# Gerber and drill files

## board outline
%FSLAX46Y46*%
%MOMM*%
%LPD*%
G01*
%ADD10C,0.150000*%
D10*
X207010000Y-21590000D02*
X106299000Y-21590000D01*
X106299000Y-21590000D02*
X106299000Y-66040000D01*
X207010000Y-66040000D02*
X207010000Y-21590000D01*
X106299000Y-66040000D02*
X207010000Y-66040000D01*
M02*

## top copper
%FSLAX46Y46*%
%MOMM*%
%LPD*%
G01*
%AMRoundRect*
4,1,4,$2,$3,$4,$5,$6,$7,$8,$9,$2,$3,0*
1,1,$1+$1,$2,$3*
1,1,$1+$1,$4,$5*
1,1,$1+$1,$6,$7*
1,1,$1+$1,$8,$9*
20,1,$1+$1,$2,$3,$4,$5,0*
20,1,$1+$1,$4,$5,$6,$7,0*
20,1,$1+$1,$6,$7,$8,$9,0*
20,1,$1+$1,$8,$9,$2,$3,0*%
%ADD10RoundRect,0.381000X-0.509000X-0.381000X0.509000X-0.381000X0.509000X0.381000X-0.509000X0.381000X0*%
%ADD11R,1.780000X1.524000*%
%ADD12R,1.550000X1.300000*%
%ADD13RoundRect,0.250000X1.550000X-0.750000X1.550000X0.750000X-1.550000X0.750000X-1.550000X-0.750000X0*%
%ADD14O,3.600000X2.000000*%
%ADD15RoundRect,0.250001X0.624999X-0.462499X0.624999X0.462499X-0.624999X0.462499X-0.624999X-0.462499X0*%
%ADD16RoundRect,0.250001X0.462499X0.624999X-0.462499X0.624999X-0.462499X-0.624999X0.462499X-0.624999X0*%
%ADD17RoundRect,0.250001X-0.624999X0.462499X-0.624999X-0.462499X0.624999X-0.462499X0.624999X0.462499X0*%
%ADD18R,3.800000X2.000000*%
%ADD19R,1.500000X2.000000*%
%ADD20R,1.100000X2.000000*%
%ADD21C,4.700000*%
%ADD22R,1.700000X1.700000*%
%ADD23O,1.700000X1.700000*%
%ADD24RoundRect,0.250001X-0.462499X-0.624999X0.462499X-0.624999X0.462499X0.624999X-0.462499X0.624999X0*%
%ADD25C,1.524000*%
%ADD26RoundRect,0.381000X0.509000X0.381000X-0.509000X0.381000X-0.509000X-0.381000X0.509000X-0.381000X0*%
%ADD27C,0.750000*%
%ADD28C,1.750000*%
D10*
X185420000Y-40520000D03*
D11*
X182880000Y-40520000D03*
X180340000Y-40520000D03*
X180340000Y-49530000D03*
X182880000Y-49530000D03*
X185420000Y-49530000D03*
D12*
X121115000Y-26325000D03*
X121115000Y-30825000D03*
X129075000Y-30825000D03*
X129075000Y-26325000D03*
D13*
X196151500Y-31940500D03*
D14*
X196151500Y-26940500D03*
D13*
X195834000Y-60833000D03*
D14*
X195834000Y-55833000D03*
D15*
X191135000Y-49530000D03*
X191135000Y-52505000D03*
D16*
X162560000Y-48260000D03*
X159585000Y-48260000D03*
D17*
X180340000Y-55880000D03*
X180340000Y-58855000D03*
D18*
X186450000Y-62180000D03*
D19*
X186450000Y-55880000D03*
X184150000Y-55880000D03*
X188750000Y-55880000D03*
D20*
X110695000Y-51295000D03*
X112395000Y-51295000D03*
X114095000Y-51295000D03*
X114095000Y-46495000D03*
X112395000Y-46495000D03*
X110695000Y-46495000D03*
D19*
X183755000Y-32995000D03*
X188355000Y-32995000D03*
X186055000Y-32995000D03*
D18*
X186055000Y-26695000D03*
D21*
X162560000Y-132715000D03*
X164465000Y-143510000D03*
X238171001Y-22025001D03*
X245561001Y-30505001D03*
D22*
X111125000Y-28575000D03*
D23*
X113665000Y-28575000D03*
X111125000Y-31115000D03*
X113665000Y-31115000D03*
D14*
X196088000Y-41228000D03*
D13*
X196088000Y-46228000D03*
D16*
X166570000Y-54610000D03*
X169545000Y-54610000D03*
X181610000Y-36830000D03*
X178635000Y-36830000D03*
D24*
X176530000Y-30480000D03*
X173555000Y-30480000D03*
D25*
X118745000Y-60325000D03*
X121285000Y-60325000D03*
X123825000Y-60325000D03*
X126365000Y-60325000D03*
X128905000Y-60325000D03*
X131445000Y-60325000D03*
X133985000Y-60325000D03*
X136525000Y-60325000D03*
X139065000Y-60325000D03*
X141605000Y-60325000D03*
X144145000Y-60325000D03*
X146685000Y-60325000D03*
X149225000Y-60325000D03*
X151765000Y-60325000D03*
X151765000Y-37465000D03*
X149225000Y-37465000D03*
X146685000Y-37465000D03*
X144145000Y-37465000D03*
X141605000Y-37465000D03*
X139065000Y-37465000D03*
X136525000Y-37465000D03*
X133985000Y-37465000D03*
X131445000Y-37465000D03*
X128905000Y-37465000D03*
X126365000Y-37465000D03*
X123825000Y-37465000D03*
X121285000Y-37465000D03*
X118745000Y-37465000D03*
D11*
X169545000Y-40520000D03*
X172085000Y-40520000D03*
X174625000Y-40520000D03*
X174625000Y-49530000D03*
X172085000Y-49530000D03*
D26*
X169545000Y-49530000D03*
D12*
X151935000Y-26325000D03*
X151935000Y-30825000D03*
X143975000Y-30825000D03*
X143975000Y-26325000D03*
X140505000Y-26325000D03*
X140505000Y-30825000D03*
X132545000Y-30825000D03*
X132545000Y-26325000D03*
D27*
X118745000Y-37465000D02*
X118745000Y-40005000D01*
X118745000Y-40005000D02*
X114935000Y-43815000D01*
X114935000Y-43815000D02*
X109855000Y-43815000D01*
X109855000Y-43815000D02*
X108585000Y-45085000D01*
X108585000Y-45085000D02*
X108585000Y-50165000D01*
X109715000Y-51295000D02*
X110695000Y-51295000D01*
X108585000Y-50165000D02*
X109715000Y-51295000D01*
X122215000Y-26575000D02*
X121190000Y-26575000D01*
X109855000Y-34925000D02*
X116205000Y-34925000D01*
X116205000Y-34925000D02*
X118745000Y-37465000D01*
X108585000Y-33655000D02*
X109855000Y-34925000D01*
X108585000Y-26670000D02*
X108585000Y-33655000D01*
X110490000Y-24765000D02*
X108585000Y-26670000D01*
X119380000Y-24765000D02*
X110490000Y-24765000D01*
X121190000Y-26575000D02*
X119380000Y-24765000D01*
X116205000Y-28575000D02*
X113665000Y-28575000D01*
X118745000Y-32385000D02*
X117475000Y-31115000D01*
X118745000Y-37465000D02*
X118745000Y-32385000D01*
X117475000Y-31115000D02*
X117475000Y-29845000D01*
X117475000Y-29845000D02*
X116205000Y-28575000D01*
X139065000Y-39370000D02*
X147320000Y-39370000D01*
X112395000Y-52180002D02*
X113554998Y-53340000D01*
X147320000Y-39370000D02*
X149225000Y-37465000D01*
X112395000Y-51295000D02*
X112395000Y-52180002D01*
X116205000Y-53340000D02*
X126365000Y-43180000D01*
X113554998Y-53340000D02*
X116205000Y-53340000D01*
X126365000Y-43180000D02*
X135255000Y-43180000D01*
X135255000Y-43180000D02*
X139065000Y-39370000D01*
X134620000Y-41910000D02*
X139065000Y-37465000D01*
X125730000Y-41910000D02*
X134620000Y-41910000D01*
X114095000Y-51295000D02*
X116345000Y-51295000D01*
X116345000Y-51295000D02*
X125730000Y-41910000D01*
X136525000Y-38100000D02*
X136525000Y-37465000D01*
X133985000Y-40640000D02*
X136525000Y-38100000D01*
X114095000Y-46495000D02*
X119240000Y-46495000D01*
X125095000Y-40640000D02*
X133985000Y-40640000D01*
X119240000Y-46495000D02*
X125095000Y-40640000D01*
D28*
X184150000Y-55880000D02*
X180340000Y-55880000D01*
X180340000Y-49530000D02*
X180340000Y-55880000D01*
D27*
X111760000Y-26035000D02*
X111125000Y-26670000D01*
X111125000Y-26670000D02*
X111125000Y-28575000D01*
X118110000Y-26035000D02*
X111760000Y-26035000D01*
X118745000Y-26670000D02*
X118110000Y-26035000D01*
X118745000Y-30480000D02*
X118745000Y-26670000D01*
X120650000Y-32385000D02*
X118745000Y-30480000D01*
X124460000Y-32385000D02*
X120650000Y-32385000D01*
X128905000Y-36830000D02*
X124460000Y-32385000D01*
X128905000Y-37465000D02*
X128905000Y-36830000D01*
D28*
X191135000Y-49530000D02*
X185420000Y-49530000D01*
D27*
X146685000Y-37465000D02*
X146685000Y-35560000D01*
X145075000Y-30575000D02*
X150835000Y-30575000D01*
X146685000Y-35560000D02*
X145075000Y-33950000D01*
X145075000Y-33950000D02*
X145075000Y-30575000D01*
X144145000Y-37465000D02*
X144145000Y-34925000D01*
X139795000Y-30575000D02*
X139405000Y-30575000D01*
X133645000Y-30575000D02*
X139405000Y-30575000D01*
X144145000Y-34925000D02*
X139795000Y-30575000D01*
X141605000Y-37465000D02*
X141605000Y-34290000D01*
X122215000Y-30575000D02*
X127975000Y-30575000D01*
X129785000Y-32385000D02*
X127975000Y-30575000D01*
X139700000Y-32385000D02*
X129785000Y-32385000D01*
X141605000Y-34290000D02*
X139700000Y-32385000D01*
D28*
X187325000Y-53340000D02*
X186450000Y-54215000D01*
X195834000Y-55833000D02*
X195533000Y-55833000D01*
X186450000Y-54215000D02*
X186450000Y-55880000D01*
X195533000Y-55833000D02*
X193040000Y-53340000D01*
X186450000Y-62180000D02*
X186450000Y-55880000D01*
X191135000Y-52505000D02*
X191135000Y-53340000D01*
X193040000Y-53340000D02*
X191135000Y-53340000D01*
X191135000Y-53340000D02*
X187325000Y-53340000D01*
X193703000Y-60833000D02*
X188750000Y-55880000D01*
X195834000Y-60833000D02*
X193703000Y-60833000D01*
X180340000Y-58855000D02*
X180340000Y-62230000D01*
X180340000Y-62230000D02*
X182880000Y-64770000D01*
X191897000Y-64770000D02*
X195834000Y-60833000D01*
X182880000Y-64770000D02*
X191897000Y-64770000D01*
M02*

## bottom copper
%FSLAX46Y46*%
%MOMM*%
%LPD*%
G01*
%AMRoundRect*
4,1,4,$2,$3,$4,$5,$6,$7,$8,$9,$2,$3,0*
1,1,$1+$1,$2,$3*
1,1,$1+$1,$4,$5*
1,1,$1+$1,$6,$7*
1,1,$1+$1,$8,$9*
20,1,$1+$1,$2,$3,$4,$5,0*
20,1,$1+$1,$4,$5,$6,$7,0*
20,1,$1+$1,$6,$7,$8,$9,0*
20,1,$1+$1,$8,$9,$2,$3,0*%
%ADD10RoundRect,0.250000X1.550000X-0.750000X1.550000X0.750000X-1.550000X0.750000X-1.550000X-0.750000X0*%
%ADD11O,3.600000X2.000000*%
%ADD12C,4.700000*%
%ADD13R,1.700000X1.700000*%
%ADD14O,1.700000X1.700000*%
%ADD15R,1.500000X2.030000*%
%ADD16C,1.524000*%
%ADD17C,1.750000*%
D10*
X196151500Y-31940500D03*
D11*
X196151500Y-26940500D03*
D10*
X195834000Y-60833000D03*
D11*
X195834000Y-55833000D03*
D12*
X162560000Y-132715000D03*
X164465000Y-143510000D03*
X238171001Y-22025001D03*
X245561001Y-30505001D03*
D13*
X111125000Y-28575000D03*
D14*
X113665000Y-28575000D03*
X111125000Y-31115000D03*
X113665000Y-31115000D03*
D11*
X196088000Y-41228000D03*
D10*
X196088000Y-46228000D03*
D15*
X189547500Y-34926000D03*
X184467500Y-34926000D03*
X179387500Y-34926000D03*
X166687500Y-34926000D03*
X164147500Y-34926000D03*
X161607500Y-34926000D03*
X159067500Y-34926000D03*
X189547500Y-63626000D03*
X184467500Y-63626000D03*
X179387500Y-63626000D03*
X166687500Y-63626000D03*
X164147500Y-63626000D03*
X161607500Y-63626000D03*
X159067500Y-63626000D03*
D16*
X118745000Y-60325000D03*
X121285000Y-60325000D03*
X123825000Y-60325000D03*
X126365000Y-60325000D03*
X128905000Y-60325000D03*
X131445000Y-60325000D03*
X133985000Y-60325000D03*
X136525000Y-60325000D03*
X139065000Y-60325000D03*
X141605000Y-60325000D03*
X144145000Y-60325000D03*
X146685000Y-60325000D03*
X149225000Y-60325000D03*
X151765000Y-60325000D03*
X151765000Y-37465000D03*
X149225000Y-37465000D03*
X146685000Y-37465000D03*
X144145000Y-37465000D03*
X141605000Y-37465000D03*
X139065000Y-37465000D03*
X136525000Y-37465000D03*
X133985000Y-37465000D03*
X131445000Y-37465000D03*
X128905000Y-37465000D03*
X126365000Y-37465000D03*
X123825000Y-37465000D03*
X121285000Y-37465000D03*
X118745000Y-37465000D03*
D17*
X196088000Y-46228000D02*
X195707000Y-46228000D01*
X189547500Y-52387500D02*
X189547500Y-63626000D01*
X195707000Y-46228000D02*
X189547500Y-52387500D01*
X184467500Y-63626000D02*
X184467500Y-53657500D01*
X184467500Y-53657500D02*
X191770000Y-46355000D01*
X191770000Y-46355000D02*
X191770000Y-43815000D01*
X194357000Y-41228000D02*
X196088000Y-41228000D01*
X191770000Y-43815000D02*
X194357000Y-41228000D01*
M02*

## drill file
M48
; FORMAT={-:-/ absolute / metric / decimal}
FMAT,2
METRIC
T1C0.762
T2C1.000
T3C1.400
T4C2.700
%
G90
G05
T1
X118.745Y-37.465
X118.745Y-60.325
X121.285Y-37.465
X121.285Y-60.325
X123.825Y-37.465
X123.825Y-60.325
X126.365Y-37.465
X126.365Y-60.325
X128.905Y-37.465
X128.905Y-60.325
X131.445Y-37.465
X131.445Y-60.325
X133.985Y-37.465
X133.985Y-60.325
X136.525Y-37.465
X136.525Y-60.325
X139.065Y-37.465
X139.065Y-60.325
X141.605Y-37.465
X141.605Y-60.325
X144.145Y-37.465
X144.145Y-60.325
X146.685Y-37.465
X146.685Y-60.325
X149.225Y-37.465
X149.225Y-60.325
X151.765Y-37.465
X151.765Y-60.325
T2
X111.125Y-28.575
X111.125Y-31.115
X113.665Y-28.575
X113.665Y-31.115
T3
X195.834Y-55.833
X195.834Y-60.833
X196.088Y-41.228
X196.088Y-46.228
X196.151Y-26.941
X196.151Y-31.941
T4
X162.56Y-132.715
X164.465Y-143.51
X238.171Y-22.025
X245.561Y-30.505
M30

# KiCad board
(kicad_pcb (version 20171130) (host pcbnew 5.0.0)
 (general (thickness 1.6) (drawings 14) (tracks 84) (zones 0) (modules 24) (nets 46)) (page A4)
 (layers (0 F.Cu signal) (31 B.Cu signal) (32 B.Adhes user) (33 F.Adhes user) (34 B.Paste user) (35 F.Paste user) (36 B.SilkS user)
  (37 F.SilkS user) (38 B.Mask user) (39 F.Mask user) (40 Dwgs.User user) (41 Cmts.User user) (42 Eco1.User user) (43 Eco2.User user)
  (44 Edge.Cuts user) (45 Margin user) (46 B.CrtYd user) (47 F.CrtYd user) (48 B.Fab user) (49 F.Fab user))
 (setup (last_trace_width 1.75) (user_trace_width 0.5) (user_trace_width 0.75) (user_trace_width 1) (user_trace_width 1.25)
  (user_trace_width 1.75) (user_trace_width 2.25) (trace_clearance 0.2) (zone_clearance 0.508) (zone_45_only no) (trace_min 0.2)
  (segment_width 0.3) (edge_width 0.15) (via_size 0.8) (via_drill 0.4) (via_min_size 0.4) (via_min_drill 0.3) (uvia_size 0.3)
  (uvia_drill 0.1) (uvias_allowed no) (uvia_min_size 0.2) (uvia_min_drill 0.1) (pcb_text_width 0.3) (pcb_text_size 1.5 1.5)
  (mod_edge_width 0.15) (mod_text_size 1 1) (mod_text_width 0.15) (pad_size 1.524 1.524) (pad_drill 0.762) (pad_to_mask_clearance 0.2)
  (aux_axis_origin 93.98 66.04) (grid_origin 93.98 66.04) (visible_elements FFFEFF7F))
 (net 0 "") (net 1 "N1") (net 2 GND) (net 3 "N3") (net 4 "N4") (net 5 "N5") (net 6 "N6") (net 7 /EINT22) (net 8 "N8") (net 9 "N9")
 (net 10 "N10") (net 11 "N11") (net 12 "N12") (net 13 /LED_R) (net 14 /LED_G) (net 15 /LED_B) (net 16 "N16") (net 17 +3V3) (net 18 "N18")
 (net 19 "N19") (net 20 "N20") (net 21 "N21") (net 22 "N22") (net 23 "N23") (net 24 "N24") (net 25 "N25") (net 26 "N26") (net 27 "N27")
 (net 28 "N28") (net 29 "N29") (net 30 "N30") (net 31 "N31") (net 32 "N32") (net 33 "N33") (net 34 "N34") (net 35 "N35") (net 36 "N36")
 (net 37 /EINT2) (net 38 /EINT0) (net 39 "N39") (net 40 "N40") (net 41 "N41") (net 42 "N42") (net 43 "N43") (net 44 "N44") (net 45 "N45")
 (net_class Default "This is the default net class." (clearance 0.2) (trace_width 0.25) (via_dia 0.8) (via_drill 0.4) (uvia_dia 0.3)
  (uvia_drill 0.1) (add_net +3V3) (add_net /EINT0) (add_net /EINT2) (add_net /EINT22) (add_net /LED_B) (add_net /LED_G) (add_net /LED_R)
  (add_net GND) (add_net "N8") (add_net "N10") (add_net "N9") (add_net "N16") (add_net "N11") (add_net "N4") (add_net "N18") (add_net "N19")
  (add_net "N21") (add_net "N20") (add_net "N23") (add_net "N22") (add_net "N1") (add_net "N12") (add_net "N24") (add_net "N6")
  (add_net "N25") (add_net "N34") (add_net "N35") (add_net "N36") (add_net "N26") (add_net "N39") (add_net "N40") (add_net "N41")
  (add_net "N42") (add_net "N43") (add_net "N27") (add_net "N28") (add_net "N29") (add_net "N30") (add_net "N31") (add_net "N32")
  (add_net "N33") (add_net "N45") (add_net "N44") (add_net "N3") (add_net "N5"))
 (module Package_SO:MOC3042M (layer F.Cu) (at 182.88 45.6 180)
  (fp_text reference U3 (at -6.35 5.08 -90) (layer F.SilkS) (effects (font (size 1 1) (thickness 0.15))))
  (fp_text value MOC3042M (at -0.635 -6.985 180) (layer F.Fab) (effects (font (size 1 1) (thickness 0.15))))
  (pad 1 smd roundrect (at -2.54 5.08) (size 1.78 1.524) (layers F.Cu F.Paste F.Mask) (roundrect_rratio 0.25) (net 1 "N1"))
  (pad 2 smd rect (at 0 5.08) (size 1.78 1.524) (layers F.Cu F.Paste F.Mask) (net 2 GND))
  (pad 3 smd rect (at 2.54 5.08) (size 1.78 1.524) (layers F.Cu F.Paste F.Mask) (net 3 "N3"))
  (pad 4 smd rect (at 2.54 -3.93) (size 1.78 1.524) (layers F.Cu F.Paste F.Mask) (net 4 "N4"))
  (pad 5 smd rect (at 0 -3.93) (size 1.78 1.524) (layers F.Cu F.Paste F.Mask) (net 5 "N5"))
  (pad 6 smd rect (at -2.54 -3.93) (size 1.78 1.524) (layers F.Cu F.Paste F.Mask) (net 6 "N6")))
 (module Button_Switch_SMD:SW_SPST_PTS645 (layer F.Cu) (at 125.095 28.575 180)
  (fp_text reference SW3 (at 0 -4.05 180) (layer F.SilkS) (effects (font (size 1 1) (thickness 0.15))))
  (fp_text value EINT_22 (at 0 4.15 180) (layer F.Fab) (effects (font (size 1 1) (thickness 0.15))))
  (pad 2 smd rect (at 3.98 2.25 180) (size 1.55 1.3) (layers F.Cu F.Paste F.Mask) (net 2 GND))
  (pad 1 smd rect (at 3.98 -2.25 180) (size 1.55 1.3) (layers F.Cu F.Paste F.Mask) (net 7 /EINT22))
  (pad 1 smd rect (at -3.98 -2.25 180) (size 1.55 1.3) (layers F.Cu F.Paste F.Mask) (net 7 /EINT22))
  (pad 2 smd rect (at -3.98 2.25 180) (size 1.55 1.3) (layers F.Cu F.Paste F.Mask) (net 2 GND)))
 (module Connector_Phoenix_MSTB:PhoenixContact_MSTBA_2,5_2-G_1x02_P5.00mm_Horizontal (layer F.Cu) (at 196.1515 31.9405 90)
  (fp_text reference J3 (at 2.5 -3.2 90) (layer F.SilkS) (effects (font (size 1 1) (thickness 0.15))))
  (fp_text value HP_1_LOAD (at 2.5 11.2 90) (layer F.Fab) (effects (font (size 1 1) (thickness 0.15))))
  (pad 1 thru_hole roundrect (at 0 0 90) (size 2 3.6) (drill 1.4) (layers *.Cu *.Mask) (roundrect_rratio 0.125) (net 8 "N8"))
  (pad 2 thru_hole oval (at 5 0 90) (size 2 3.6) (drill 1.4) (layers *.Cu *.Mask) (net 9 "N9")))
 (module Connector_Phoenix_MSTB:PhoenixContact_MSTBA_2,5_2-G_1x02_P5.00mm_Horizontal (layer F.Cu) (at 195.834 60.833 90)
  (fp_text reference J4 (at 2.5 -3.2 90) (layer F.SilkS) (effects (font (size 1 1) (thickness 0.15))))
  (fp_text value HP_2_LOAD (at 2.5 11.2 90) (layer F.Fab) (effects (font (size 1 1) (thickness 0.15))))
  (pad 1 thru_hole roundrect (at 0 0 90) (size 2 3.6) (drill 1.4) (layers *.Cu *.Mask) (roundrect_rratio 0.125) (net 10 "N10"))
  (pad 2 thru_hole oval (at 5 0 90) (size 2 3.6) (drill 1.4) (layers *.Cu *.Mask) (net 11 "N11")))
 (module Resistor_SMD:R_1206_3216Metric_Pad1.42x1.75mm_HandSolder (layer F.Cu) (at 191.135 51.0175 90)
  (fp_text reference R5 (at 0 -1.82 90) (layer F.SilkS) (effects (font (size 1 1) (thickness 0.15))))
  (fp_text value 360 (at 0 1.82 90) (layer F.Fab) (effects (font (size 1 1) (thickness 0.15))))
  (pad 2 smd roundrect (at 1.4875 0 90) (size 1.425 1.75) (layers F.Cu F.Paste F.Mask) (roundrect_rratio 0.175439) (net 6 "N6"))
  (pad 1 smd roundrect (at -1.4875 0 90) (size 1.425 1.75) (layers F.Cu F.Paste F.Mask) (roundrect_rratio 0.175439) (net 11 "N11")))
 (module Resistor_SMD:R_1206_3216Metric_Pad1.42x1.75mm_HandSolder (layer F.Cu) (at 161.0725 48.26 180)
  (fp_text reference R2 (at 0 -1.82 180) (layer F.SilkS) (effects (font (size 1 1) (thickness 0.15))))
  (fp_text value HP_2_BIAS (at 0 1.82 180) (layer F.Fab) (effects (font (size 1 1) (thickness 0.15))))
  (pad 1 smd roundrect (at -1.4875 0 180) (size 1.425 1.75) (layers F.Cu F.Paste F.Mask) (roundrect_rratio 0.175439) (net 1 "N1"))
  (pad 2 smd roundrect (at 1.4875 0 180) (size 1.425 1.75) (layers F.Cu F.Paste F.Mask) (roundrect_rratio 0.175439) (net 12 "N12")))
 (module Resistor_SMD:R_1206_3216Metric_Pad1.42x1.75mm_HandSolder (layer F.Cu) (at 180.34 57.3675 270)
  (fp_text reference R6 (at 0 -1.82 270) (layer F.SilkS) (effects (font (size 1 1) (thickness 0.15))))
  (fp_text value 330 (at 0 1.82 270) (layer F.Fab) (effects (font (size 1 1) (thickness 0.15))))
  (pad 1 smd roundrect (at -1.4875 0 270) (size 1.425 1.75) (layers F.Cu F.Paste F.Mask) (roundrect_rratio 0.175439) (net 4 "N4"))
  (pad 2 smd roundrect (at 1.4875 0 270) (size 1.425 1.75) (layers F.Cu F.Paste F.Mask) (roundrect_rratio 0.175439) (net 10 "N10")))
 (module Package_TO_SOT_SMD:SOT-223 (layer F.Cu) (at 186.45 59.03 270)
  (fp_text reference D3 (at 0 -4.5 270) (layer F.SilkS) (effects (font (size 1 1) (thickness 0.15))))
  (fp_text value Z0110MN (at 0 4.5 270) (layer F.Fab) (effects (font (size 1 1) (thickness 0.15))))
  (pad 4 smd rect (at 3.15 0 270) (size 2 3.8) (layers F.Cu F.Paste F.Mask) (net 11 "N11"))
  (pad 2 smd rect (at -3.15 0 270) (size 2 1.5) (layers F.Cu F.Paste F.Mask) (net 11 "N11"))
  (pad 3 smd rect (at -3.15 2.3 270) (size 2 1.5) (layers F.Cu F.Paste F.Mask) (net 4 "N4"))
  (pad 1 smd rect (at -3.15 -2.3 270) (size 2 1.5) (layers F.Cu F.Paste F.Mask) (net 10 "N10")))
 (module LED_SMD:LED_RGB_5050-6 (layer F.Cu) (at 112.395 48.895 90)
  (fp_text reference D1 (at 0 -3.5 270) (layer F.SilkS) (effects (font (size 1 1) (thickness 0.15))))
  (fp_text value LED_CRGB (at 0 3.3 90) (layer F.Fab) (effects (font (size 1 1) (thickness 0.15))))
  (pad 1 smd rect (at -2.4 -1.7 180) (size 1.1 2) (layers F.Cu F.Paste F.Mask) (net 2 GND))
  (pad 2 smd rect (at -2.4 0 180) (size 1.1 2) (layers F.Cu F.Paste F.Mask) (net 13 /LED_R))
  (pad 3 smd rect (at -2.4 1.7 180) (size 1.1 2) (layers F.Cu F.Paste F.Mask) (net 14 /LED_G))
  (pad 4 smd rect (at 2.4 1.7 180) (size 1.1 2) (layers F.Cu F.Paste F.Mask) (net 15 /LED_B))
  (pad 5 smd rect (at 2.4 0 180) (size 1.1 2) (layers F.Cu F.Paste F.Mask))
  (pad 6 smd rect (at 2.4 -1.7 180) (size 1.1 2) (layers F.Cu F.Paste F.Mask)))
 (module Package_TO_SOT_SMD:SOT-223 (layer F.Cu) (at 186.055 29.845 90)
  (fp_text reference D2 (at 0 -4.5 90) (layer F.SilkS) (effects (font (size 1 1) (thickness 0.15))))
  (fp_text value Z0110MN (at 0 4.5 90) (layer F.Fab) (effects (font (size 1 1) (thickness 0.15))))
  (pad 1 smd rect (at -3.15 -2.3 90) (size 2 1.5) (layers F.Cu F.Paste F.Mask) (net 8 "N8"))
  (pad 3 smd rect (at -3.15 2.3 90) (size 2 1.5) (layers F.Cu F.Paste F.Mask) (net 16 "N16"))
  (pad 2 smd rect (at -3.15 0 90) (size 2 1.5) (layers F.Cu F.Paste F.Mask) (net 9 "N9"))
  (pad 4 smd rect (at 3.15 0 90) (size 2 3.8) (layers F.Cu F.Paste F.Mask) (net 9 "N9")))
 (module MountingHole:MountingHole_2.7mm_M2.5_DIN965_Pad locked (layer F.Cu) (at 162.56 132.715)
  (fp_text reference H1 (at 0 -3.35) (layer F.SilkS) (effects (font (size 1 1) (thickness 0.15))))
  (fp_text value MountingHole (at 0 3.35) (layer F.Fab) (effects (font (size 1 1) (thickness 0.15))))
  (pad 1 thru_hole circle (at 0 0) (size 4.7 4.7) (drill 2.7) (layers *.Cu *.Mask)))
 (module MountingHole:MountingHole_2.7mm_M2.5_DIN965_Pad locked (layer F.Cu) (at 164.465 143.51)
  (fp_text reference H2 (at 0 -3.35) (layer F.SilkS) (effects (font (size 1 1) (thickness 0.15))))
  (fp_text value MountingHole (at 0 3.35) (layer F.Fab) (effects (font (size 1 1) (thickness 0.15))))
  (pad 1 thru_hole circle (at 0 0) (size 4.7 4.7) (drill 2.7) (layers *.Cu *.Mask)))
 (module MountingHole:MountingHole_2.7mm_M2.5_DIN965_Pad (layer F.Cu) (at 238.171001 22.025001)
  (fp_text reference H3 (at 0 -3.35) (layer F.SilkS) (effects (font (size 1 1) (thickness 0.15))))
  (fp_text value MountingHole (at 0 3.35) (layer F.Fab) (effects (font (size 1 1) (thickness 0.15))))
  (pad 1 thru_hole circle (at 0 0) (size 4.7 4.7) (drill 2.7) (layers *.Cu *.Mask)))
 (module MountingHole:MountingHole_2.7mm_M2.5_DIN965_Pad (layer F.Cu) (at 245.561001 30.505001)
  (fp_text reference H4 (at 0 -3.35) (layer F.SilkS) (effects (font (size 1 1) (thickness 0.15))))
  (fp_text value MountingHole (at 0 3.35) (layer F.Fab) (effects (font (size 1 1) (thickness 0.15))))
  (pad 1 thru_hole circle (at 0 0) (size 4.7 4.7) (drill 2.7) (layers *.Cu *.Mask)))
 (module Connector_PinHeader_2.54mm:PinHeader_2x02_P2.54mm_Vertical (layer F.Cu) (at 111.125 28.575)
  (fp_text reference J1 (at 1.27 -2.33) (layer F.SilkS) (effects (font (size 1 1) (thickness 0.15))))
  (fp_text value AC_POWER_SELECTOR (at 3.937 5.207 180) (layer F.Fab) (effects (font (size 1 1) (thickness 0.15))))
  (pad 1 thru_hole rect (at 0 0) (size 1.7 1.7) (drill 1) (layers *.Cu *.Mask) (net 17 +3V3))
  (pad 2 thru_hole oval (at 2.54 0) (size 1.7 1.7) (drill 1) (layers *.Cu *.Mask) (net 2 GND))
  (pad 3 thru_hole oval (at 0 2.54) (size 1.7 1.7) (drill 1) (layers *.Cu *.Mask) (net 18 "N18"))
  (pad 4 thru_hole oval (at 2.54 2.54) (size 1.7 1.7) (drill 1) (layers *.Cu *.Mask) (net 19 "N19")))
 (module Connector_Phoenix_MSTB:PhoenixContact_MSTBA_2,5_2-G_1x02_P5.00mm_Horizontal (layer F.Cu) (at 196.088 46.228 90)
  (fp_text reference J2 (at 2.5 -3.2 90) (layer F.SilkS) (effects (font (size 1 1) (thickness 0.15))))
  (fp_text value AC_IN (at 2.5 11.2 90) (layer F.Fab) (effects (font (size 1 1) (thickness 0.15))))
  (pad 2 thru_hole oval (at 5 0 90) (size 2 3.6) (drill 1.4) (layers *.Cu *.Mask) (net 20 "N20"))
  (pad 1 thru_hole roundrect (at 0 0 90) (size 2 3.6) (drill 1.4) (layers *.Cu *.Mask) (roundrect_rratio 0.125) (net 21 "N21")))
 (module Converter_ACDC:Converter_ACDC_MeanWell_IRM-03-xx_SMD (layer B.Cu) (at 174.3075 49.276 90)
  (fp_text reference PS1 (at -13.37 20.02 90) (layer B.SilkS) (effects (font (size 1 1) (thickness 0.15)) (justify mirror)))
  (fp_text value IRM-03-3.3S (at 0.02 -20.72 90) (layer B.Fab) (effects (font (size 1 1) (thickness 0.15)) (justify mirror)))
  (pad 26 smd rect (at 14.35 15.24 180) (size 1.5 2.03) (layers B.Cu B.Paste B.Mask))
  (pad 24 smd rect (at 14.35 10.16 180) (size 1.5 2.03) (layers B.Cu B.Paste B.Mask))
  (pad 22 smd rect (at 14.35 5.08 180) (size 1.5 2.03) (layers B.Cu B.Paste B.Mask))
  (pad 17 smd rect (at 14.35 -7.62 180) (size 1.5 2.03) (layers B.Cu B.Paste B.Mask))
  (pad 16 smd rect (at 14.35 -10.16 180) (size 1.5 2.03) (layers B.Cu B.Paste B.Mask) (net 19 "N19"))
  (pad 15 smd rect (at 14.35 -12.7 180) (size 1.5 2.03) (layers B.Cu B.Paste B.Mask))
  (pad 14 smd rect (at 14.35 -15.24 180) (size 1.5 2.03) (layers B.Cu B.Paste B.Mask) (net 18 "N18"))
  (pad 1 smd rect (at -14.35 15.24 180) (size 1.5 2.03) (layers B.Cu B.Paste B.Mask) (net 21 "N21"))
  (pad 3 smd rect (at -14.35 10.16 180) (size 1.5 2.03) (layers B.Cu B.Paste B.Mask) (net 20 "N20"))
  (pad 5 smd rect (at -14.35 5.08 180) (size 1.5 2.03) (layers B.Cu B.Paste B.Mask))
  (pad 10 smd rect (at -14.35 -7.62 180) (size 1.5 2.03) (layers B.Cu B.Paste B.Mask))
  (pad 11 smd rect (at -14.35 -10.16 180) (size 1.5 2.03) (layers B.Cu B.Paste B.Mask))
  (pad 12 smd rect (at -14.35 -12.7 180) (size 1.5 2.03) (layers B.Cu B.Paste B.Mask))
  (pad 13 smd rect (at -14.35 -15.24 180) (size 1.5 2.03) (layers B.Cu B.Paste B.Mask)))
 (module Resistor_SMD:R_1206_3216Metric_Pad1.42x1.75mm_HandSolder (layer F.Cu) (at 168.0575 54.61 180)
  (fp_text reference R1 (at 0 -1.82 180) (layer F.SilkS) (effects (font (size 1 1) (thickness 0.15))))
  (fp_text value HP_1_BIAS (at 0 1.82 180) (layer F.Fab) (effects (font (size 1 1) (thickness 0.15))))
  (pad 2 smd roundrect (at 1.4875 0 180) (size 1.425 1.75) (layers F.Cu F.Paste F.Mask) (roundrect_rratio 0.175439) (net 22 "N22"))
  (pad 1 smd roundrect (at -1.4875 0 180) (size 1.425 1.75) (layers F.Cu F.Paste F.Mask) (roundrect_rratio 0.175439) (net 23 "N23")))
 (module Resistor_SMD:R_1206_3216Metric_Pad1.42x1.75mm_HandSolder (layer F.Cu) (at 180.1225 36.83 180)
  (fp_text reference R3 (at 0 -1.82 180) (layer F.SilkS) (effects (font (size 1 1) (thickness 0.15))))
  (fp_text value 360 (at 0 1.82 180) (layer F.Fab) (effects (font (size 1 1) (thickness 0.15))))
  (pad 1 smd roundrect (at -1.4875 0 180) (size 1.425 1.75) (layers F.Cu F.Paste F.Mask) (roundrect_rratio 0.175439) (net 9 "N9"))
  (pad 2 smd roundrect (at 1.4875 0 180) (size 1.425 1.75) (layers F.Cu F.Paste F.Mask) (roundrect_rratio 0.175439) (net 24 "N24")))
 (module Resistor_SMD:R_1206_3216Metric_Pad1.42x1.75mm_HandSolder (layer F.Cu) (at 175.0425 30.48)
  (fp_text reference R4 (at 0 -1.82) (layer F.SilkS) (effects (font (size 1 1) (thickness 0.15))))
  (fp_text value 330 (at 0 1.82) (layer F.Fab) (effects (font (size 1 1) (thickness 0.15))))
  (pad 2 smd roundrect (at 1.4875 0) (size 1.425 1.75) (layers F.Cu F.Paste F.Mask) (roundrect_rratio 0.175439) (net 8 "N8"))
  (pad 1 smd roundrect (at -1.4875 0) (size 1.425 1.75) (layers F.Cu F.Paste F.Mask) (roundrect_rratio 0.175439) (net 16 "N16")))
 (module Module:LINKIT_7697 (layer F.Cu) (at 151.765 37.465 180)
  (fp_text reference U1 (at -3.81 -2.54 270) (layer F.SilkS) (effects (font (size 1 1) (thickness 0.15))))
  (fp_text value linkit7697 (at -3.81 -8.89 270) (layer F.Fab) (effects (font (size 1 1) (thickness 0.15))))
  (pad 1 thru_hole circle (at 33.02 -22.86 180) (size 1.524 1.524) (drill 0.762) (layers *.Cu *.Mask) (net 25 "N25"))
  (pad 2 thru_hole circle (at 30.48 -22.86 180) (size 1.524 1.524) (drill 0.762) (layers *.Cu *.Mask) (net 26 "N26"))
  (pad 3 thru_hole circle (at 27.94 -22.86 180) (size 1.524 1.524) (drill 0.762) (layers *.Cu *.Mask) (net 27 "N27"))
  (pad 4 thru_hole circle (at 25.4 -22.86 180) (size 1.524 1.524) (drill 0.762) (layers *.Cu *.Mask) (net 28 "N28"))
  (pad 5 thru_hole circle (at 22.86 -22.86 180) (size 1.524 1.524) (drill 0.762) (layers *.Cu *.Mask) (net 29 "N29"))
  (pad 6 thru_hole circle (at 20.32 -22.86 180) (size 1.524 1.524) (drill 0.762) (layers *.Cu *.Mask) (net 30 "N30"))
  (pad 7 thru_hole circle (at 17.78 -22.86 180) (size 1.524 1.524) (drill 0.762) (layers *.Cu *.Mask) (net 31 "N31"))
  (pad 8 thru_hole circle (at 15.24 -22.86 180) (size 1.524 1.524) (drill 0.762) (layers *.Cu *.Mask) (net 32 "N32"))
  (pad 9 thru_hole circle (at 12.7 -22.86 180) (size 1.524 1.524) (drill 0.762) (layers *.Cu *.Mask) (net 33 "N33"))
  (pad 10 thru_hole circle (at 10.16 -22.86 180) (size 1.524 1.524) (drill 0.762) (layers *.Cu *.Mask) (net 12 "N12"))
  (pad 11 thru_hole circle (at 7.62 -22.86 180) (size 1.524 1.524) (drill 0.762) (layers *.Cu *.Mask) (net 22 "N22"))
  (pad 12 thru_hole circle (at 5.08 -22.86 180) (size 1.524 1.524) (drill 0.762) (layers *.Cu *.Mask) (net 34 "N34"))
  (pad 13 thru_hole circle (at 2.54 -22.86 180) (size 1.524 1.524) (drill 0.762) (layers *.Cu *.Mask) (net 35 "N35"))
  (pad 14 thru_hole circle (at 0 -22.86 180) (size 1.524 1.524) (drill 0.762) (layers *.Cu *.Mask) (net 17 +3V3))
  (pad 15 thru_hole circle (at 0 0 180) (size 1.524 1.524) (drill 0.762) (layers *.Cu *.Mask) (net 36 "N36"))
  (pad 16 thru_hole circle (at 2.54 0 180) (size 1.524 1.524) (drill 0.762) (layers *.Cu *.Mask) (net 13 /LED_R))
  (pad 17 thru_hole circle (at 5.08 0 180) (size 1.524 1.524) (drill 0.762) (layers *.Cu *.Mask) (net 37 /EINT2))
  (pad 18 thru_hole circle (at 7.62 0 180) (size 1.524 1.524) (drill 0.762) (layers *.Cu *.Mask) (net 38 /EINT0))
  (pad 19 thru_hole circle (at 10.16 0 180) (size 1.524 1.524) (drill 0.762) (layers *.Cu *.Mask) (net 7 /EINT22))
  (pad 20 thru_hole circle (at 12.7 0 180) (size 1.524 1.524) (drill 0.762) (layers *.Cu *.Mask) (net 14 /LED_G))
  (pad 21 thru_hole circle (at 15.24 0 180) (size 1.524 1.524) (drill 0.762) (layers *.Cu *.Mask) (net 15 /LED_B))
  (pad 22 thru_hole circle (at 17.78 0 180) (size 1.524 1.524) (drill 0.762) (layers *.Cu *.Mask) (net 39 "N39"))
  (pad 23 thru_hole circle (at 20.32 0 180) (size 1.524 1.524) (drill 0.762) (layers *.Cu *.Mask) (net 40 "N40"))
  (pad 24 thru_hole circle (at 22.86 0 180) (size 1.524 1.524) (drill 0.762) (layers *.Cu *.Mask) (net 17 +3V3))
  (pad 25 thru_hole circle (at 25.4 0 180) (size 1.524 1.524) (drill 0.762) (layers *.Cu *.Mask) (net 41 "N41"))
  (pad 26 thru_hole circle (at 27.94 0 180) (size 1.524 1.524) (drill 0.762) (layers *.Cu *.Mask) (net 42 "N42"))
  (pad 27 thru_hole circle (at 30.48 0 180) (size 1.524 1.524) (drill 0.762) (layers *.Cu *.Mask) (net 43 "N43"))
  (pad 28 thru_hole circle (at 33.02 0 180) (size 1.524 1.524) (drill 0.762) (layers *.Cu *.Mask) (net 2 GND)))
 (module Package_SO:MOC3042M (layer F.Cu) (at 172.085 44.45)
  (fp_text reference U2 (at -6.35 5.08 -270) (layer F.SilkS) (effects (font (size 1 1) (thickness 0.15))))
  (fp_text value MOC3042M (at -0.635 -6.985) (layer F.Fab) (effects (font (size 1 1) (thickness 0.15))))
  (pad 6 smd rect (at -2.54 -3.93 180) (size 1.78 1.524) (layers F.Cu F.Paste F.Mask) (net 24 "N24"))
  (pad 5 smd rect (at 0 -3.93 180) (size 1.78 1.524) (layers F.Cu F.Paste F.Mask) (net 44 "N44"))
  (pad 4 smd rect (at 2.54 -3.93 180) (size 1.78 1.524) (layers F.Cu F.Paste F.Mask) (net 16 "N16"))
  (pad 3 smd rect (at 2.54 5.08 180) (size 1.78 1.524) (layers F.Cu F.Paste F.Mask) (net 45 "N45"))
  (pad 2 smd rect (at 0 5.08 180) (size 1.78 1.524) (layers F.Cu F.Paste F.Mask) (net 2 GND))
  (pad 1 smd roundrect (at -2.54 5.08 180) (size 1.78 1.524) (layers F.Cu F.Paste F.Mask) (roundrect_rratio 0.25) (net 23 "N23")))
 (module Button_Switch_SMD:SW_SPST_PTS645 (layer F.Cu) (at 147.955 28.575 180)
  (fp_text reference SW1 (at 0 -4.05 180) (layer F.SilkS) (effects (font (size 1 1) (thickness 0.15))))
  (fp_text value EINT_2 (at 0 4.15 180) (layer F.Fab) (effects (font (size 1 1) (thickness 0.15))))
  (pad 2 smd rect (at -3.98 2.25 180) (size 1.55 1.3) (layers F.Cu F.Paste F.Mask) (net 2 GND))
  (pad 1 smd rect (at -3.98 -2.25 180) (size 1.55 1.3) (layers F.Cu F.Paste F.Mask) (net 37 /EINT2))
  (pad 1 smd rect (at 3.98 -2.25 180) (size 1.55 1.3) (layers F.Cu F.Paste F.Mask) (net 37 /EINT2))
  (pad 2 smd rect (at 3.98 2.25 180) (size 1.55 1.3) (layers F.Cu F.Paste F.Mask) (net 2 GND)))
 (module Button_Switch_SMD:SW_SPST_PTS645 (layer F.Cu) (at 136.525 28.575 180)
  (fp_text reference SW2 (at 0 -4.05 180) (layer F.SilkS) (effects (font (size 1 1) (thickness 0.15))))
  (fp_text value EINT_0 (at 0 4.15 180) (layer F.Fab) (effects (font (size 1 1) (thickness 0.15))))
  (pad 2 smd rect (at -3.98 2.25 180) (size 1.55 1.3) (layers F.Cu F.Paste F.Mask) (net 2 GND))
  (pad 1 smd rect (at -3.98 -2.25 180) (size 1.55 1.3) (layers F.Cu F.Paste F.Mask) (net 38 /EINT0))
  (pad 1 smd rect (at 3.98 -2.25 180) (size 1.55 1.3) (layers F.Cu F.Paste F.Mask) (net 38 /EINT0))
  (pad 2 smd rect (at 3.98 2.25 180) (size 1.55 1.3) (layers F.Cu F.Paste F.Mask) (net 2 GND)))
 (gr_line (start 207.01 21.59) (end 106.299 21.59) (layer Edge.Cuts) (width 0.15))
 (gr_line (start 106.299 21.59) (end 106.299 66.04) (layer Edge.Cuts) (width 0.15))
 (gr_line (start 207.01 66.04) (end 207.01 21.59) (layer Edge.Cuts) (width 0.15))
 (gr_line (start 106.299 66.04) (end 207.01 66.04) (layer Edge.Cuts) (width 0.15))
 (segment (start 118.745 37.465) (end 118.745 40.005) (width 0.75) (layer F.Cu) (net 2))
 (segment (start 118.745 40.005) (end 114.935 43.815) (width 0.75) (layer F.Cu) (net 2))
 (segment (start 114.935 43.815) (end 109.855 43.815) (width 0.75) (layer F.Cu) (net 2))
 (segment (start 109.855 43.815) (end 108.585 45.085) (width 0.75) (layer F.Cu) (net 2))
 (segment (start 108.585 45.085) (end 108.585 50.165) (width 0.75) (layer F.Cu) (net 2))
 (segment (start 109.715 51.295) (end 110.695 51.295) (width 0.75) (layer F.Cu) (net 2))
 (segment (start 108.585 50.165) (end 109.715 51.295) (width 0.75) (layer F.Cu) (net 2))
 (segment (start 122.215 26.575) (end 121.19 26.575) (width 0.75) (layer F.Cu) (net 2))
 (segment (start 109.855 34.925) (end 116.205 34.925) (width 0.75) (layer F.Cu) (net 2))
 (segment (start 116.205 34.925) (end 118.745 37.465) (width 0.75) (layer F.Cu) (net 2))
 (segment (start 108.585 33.655) (end 109.855 34.925) (width 0.75) (layer F.Cu) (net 2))
 (segment (start 108.585 26.67) (end 108.585 33.655) (width 0.75) (layer F.Cu) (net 2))
 (segment (start 110.49 24.765) (end 108.585 26.67) (width 0.75) (layer F.Cu) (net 2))
 (segment (start 119.38 24.765) (end 110.49 24.765) (width 0.75) (layer F.Cu) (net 2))
 (segment (start 121.19 26.575) (end 119.38 24.765) (width 0.75) (layer F.Cu) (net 2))
 (segment (start 116.205 28.575) (end 113.665 28.575) (width 0.75) (layer F.Cu) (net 2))
 (segment (start 118.745 32.385) (end 117.475 31.115) (width 0.75) (layer F.Cu) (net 2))
 (segment (start 118.745 37.465) (end 118.745 32.385) (width 0.75) (layer F.Cu) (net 2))
 (segment (start 117.475 31.115) (end 117.475 29.845) (width 0.75) (layer F.Cu) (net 2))
 (segment (start 117.475 29.845) (end 116.205 28.575) (width 0.75) (layer F.Cu) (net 2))
 (segment (start 139.065 39.37) (end 147.32 39.37) (width 0.75) (layer F.Cu) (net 13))
 (segment (start 112.395 52.180002) (end 113.554998 53.34) (width 0.75) (layer F.Cu) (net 13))
 (segment (start 147.32 39.37) (end 149.225 37.465) (width 0.75) (layer F.Cu) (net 13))
 (segment (start 112.395 51.295) (end 112.395 52.180002) (width 0.75) (layer F.Cu) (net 13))
 (segment (start 116.205 53.34) (end 126.365 43.18) (width 0.75) (layer F.Cu) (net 13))
 (segment (start 113.554998 53.34) (end 116.205 53.34) (width 0.75) (layer F.Cu) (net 13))
 (segment (start 126.365 43.18) (end 135.255 43.18) (width 0.75) (layer F.Cu) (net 13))
 (segment (start 135.255 43.18) (end 139.065 39.37) (width 0.75) (layer F.Cu) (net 13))
 (segment (start 134.62 41.91) (end 139.065 37.465) (width 0.75) (layer F.Cu) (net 14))
 (segment (start 125.73 41.91) (end 134.62 41.91) (width 0.75) (layer F.Cu) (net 14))
 (segment (start 114.095 51.295) (end 116.345 51.295) (width 0.75) (layer F.Cu) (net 14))
 (segment (start 116.345 51.295) (end 125.73 41.91) (width 0.75) (layer F.Cu) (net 14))
 (segment (start 136.525 38.1) (end 136.525 37.465) (width 0.75) (layer F.Cu) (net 15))
 (segment (start 133.985 40.64) (end 136.525 38.1) (width 0.75) (layer F.Cu) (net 15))
 (segment (start 114.095 46.495) (end 119.24 46.495) (width 0.75) (layer F.Cu) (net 15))
 (segment (start 125.095 40.64) (end 133.985 40.64) (width 0.75) (layer F.Cu) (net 15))
 (segment (start 119.24 46.495) (end 125.095 40.64) (width 0.75) (layer F.Cu) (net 15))
 (segment (start 184.15 55.88) (end 180.34 55.88) (width 1.75) (layer F.Cu) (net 4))
 (segment (start 180.34 49.53) (end 180.34 55.88) (width 1.75) (layer F.Cu) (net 4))
 (segment (start 111.76 26.035) (end 111.125 26.67) (width 0.75) (layer F.Cu) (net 17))
 (segment (start 111.125 26.67) (end 111.125 28.575) (width 0.75) (layer F.Cu) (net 17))
 (segment (start 118.11 26.035) (end 111.76 26.035) (width 0.75) (layer F.Cu) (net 17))
 (segment (start 118.745 26.67) (end 118.11 26.035) (width 0.75) (layer F.Cu) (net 17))
 (segment (start 118.745 30.48) (end 118.745 26.67) (width 0.75) (layer F.Cu) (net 17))
 (segment (start 120.65 32.385) (end 118.745 30.48) (width 0.75) (layer F.Cu) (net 17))
 (segment (start 124.46 32.385) (end 120.65 32.385) (width 0.75) (layer F.Cu) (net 17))
 (segment (start 128.905 36.83) (end 124.46 32.385) (width 0.75) (layer F.Cu) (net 17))
 (segment (start 128.905 37.465) (end 128.905 36.83) (width 0.75) (layer F.Cu) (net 17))
 (segment (start 196.088 46.228) (end 195.707 46.228) (width 1.75) (layer B.Cu) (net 21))
 (segment (start 189.5475 52.3875) (end 189.5475 63.626) (width 1.75) (layer B.Cu) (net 21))
 (segment (start 195.707 46.228) (end 189.5475 52.3875) (width 1.75) (layer B.Cu) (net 21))
 (segment (start 184.4675 63.626) (end 184.4675 53.6575) (width 1.75) (layer B.Cu) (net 20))
 (segment (start 184.4675 53.6575) (end 191.77 46.355) (width 1.75) (layer B.Cu) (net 20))
 (segment (start 191.77 46.355) (end 191.77 43.815) (width 1.75) (layer B.Cu) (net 20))
 (segment (start 194.357 41.228) (end 196.088 41.228) (width 1.75) (layer B.Cu) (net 20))
 (segment (start 191.77 43.815) (end 194.357 41.228) (width 1.75) (layer B.Cu) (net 20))
 (segment (start 191.135 49.53) (end 185.42 49.53) (width 1.75) (layer F.Cu) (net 6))
 (segment (start 146.685 37.465) (end 146.685 35.56) (width 0.75) (layer F.Cu) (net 37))
 (segment (start 145.075 30.575) (end 150.835 30.575) (width 0.75) (layer F.Cu) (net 37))
 (segment (start 146.685 35.56) (end 145.075 33.95) (width 0.75) (layer F.Cu) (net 37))
 (segment (start 145.075 33.95) (end 145.075 30.575) (width 0.75) (layer F.Cu) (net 37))
 (segment (start 144.145 37.465) (end 144.145 34.925) (width 0.75) (layer F.Cu) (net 38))
 (segment (start 139.795 30.575) (end 139.405 30.575) (width 0.75) (layer F.Cu) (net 38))
 (segment (start 133.645 30.575) (end 139.405 30.575) (width 0.75) (layer F.Cu) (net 38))
 (segment (start 144.145 34.925) (end 139.795 30.575) (width 0.75) (layer F.Cu) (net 38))
 (segment (start 141.605 37.465) (end 141.605 34.29) (width 0.75) (layer F.Cu) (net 7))
 (segment (start 122.215 30.575) (end 127.975 30.575) (width 0.75) (layer F.Cu) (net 7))
 (segment (start 129.785 32.385) (end 127.975 30.575) (width 0.75) (layer F.Cu) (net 7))
 (segment (start 139.7 32.385) (end 129.785 32.385) (width 0.75) (layer F.Cu) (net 7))
 (segment (start 141.605 34.29) (end 139.7 32.385) (width 0.75) (layer F.Cu) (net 7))
 (segment (start 187.325 53.34) (end 186.45 54.215) (width 1.75) (layer F.Cu) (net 11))
 (segment (start 195.834 55.833) (end 195.533 55.833) (width 1.75) (layer F.Cu) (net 11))
 (segment (start 186.45 54.215) (end 186.45 55.88) (width 1.75) (layer F.Cu) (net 11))
 (segment (start 195.533 55.833) (end 193.04 53.34) (width 1.75) (layer F.Cu) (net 11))
 (segment (start 186.45 62.18) (end 186.45 55.88) (width 1.75) (layer F.Cu) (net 11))
 (segment (start 191.135 52.505) (end 191.135 53.34) (width 1.75) (layer F.Cu) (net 11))
 (segment (start 193.04 53.34) (end 191.135 53.34) (width 1.75) (layer F.Cu) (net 11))
 (segment (start 191.135 53.34) (end 187.325 53.34) (width 1.75) (layer F.Cu) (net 11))
 (segment (start 193.703 60.833) (end 188.75 55.88) (width 1.75) (layer F.Cu) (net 10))
 (segment (start 195.834 60.833) (end 193.703 60.833) (width 1.75) (layer F.Cu) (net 10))
 (segment (start 180.34 58.855) (end 180.34 62.23) (width 1.75) (layer F.Cu) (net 10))
 (segment (start 180.34 62.23) (end 182.88 64.77) (width 1.75) (layer F.Cu) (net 10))
 (segment (start 191.897 64.77) (end 195.834 60.833) (width 1.75) (layer F.Cu) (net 10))
 (segment (start 182.88 64.77) (end 191.897 64.77) (width 1.75) (layer F.Cu) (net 10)))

